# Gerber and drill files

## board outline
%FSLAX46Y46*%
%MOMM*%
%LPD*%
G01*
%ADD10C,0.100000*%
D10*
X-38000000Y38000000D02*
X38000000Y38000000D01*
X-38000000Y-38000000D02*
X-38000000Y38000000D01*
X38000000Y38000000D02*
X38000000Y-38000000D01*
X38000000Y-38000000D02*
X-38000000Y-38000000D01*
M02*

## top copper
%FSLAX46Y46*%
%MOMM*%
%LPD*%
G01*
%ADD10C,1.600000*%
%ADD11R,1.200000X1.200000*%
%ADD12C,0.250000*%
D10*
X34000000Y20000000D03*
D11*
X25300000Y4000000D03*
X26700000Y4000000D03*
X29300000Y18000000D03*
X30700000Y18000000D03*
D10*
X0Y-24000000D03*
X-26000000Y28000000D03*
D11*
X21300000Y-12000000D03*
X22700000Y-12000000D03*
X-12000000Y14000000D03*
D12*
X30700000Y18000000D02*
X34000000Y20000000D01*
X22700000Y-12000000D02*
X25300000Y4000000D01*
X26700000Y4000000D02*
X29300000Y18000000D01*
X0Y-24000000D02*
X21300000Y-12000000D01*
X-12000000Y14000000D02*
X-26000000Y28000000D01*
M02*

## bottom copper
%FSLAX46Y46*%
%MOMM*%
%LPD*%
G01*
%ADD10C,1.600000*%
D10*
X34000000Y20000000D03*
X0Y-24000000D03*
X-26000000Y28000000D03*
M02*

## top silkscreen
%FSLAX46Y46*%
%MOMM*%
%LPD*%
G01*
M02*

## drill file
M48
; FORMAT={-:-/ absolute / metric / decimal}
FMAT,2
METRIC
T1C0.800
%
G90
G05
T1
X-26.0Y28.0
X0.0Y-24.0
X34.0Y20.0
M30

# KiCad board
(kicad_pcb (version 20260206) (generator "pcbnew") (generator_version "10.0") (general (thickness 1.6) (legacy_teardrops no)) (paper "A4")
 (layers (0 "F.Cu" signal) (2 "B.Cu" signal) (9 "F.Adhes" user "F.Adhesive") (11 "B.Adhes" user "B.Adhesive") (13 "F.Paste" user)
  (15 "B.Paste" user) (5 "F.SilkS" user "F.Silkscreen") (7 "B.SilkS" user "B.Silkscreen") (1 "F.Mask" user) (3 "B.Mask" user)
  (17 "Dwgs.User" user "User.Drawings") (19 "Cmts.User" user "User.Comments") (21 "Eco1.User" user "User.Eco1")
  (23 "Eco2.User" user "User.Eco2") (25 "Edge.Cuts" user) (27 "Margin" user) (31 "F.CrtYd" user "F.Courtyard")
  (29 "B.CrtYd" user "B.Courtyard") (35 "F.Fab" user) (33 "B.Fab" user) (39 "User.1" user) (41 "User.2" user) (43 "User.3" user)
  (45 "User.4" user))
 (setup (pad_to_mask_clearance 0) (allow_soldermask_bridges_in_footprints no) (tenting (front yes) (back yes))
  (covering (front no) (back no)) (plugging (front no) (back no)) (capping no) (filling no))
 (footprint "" (layer "F.Cu") (at 34 -20)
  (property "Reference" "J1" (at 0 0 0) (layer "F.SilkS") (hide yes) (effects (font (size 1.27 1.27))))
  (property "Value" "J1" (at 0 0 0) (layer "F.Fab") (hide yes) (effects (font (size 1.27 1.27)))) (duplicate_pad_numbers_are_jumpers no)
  (pad "1" thru_hole circle (at 0 0) (size 1.6 1.6) (drill 0.8) (layers "*.Cu" "*.Mask") (remove_unused_layers no) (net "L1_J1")))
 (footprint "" (layer "F.Cu") (at 26 -4)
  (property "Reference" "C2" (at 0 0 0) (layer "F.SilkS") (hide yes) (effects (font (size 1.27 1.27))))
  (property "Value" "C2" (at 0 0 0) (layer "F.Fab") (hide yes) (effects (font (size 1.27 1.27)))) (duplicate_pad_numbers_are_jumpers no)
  (pad "1" smd rect (at -0.7 0) (size 1.2 1.2) (layers "F.Cu" "F.Mask" "F.Paste") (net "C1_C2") (thermal_bridge_angle 45))
  (pad "2" smd rect (at 0.7 0) (size 1.2 1.2) (layers "F.Cu" "F.Mask" "F.Paste") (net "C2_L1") (thermal_bridge_angle 45)))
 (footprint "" (layer "F.Cu") (at 30 -18)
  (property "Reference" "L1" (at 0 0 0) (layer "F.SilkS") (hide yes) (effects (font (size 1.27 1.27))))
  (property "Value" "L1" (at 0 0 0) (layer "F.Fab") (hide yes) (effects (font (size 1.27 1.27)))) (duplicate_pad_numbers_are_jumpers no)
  (pad "1" smd rect (at -0.7 0) (size 1.2 1.2) (layers "F.Cu" "F.Mask" "F.Paste") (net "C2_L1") (thermal_bridge_angle 45))
  (pad "2" smd rect (at 0.7 0) (size 1.2 1.2) (layers "F.Cu" "F.Mask" "F.Paste") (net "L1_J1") (thermal_bridge_angle 45)))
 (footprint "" (layer "F.Cu") (at 0 24)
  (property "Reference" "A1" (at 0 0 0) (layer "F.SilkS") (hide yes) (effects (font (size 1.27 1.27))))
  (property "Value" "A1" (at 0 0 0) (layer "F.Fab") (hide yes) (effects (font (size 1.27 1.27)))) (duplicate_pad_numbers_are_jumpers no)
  (pad "1" thru_hole circle (at 0 0) (size 1.6 1.6) (drill 0.8) (layers "*.Cu" "*.Mask") (remove_unused_layers no) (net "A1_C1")))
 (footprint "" (layer "F.Cu") (at -26 -28)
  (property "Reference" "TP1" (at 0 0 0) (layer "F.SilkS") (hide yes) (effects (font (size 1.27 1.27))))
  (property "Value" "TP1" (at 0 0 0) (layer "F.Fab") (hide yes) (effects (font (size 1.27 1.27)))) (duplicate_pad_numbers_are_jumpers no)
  (pad "1" thru_hole circle (at 0 0) (size 1.6 1.6) (drill 0.8) (layers "*.Cu" "*.Mask") (remove_unused_layers no) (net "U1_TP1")))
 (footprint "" (layer "F.Cu") (at 22 12)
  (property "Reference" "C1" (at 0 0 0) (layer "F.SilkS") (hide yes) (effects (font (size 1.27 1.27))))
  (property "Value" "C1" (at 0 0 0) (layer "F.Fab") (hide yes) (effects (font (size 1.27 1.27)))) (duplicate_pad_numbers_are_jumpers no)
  (pad "1" smd rect (at -0.7 0) (size 1.2 1.2) (layers "F.Cu" "F.Mask" "F.Paste") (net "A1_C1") (thermal_bridge_angle 45))
  (pad "2" smd rect (at 0.7 0) (size 1.2 1.2) (layers "F.Cu" "F.Mask" "F.Paste") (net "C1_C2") (thermal_bridge_angle 45)))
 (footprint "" (layer "F.Cu") (at -12 -14)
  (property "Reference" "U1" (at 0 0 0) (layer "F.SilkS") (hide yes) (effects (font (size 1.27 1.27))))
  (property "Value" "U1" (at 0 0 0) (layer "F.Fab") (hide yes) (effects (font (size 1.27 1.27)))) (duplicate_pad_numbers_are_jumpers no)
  (pad "1" smd rect (at 0 0) (size 1.2 1.2) (layers "F.Cu" "F.Mask" "F.Paste") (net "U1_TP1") (thermal_bridge_angle 45)))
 (gr_line (start -38 -38) (end 38 -38) (stroke (width 0.1) (type default)) (layer "Edge.Cuts"))
 (gr_line (start -38 38) (end -38 -38) (stroke (width 0.1) (type default)) (layer "Edge.Cuts"))
 (gr_line (start 38 -38) (end 38 38) (stroke (width 0.1) (type default)) (layer "Edge.Cuts"))
 (gr_line (start 38 38) (end -38 38) (stroke (width 0.1) (type default)) (layer "Edge.Cuts"))
 (segment (start 30.7 -18) (end 34 -20) (width 0.25) (layer "F.Cu") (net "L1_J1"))
 (segment (start 22.7 12) (end 25.3 -4) (width 0.25) (layer "F.Cu") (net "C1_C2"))
 (segment (start 26.7 -4) (end 29.3 -18) (width 0.25) (layer "F.Cu") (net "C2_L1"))
 (segment (start 0 24) (end 21.3 12) (width 0.25) (layer "F.Cu") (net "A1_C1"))
 (segment (start -12 -14) (end -26 -28) (width 0.25) (layer "F.Cu") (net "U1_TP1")))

